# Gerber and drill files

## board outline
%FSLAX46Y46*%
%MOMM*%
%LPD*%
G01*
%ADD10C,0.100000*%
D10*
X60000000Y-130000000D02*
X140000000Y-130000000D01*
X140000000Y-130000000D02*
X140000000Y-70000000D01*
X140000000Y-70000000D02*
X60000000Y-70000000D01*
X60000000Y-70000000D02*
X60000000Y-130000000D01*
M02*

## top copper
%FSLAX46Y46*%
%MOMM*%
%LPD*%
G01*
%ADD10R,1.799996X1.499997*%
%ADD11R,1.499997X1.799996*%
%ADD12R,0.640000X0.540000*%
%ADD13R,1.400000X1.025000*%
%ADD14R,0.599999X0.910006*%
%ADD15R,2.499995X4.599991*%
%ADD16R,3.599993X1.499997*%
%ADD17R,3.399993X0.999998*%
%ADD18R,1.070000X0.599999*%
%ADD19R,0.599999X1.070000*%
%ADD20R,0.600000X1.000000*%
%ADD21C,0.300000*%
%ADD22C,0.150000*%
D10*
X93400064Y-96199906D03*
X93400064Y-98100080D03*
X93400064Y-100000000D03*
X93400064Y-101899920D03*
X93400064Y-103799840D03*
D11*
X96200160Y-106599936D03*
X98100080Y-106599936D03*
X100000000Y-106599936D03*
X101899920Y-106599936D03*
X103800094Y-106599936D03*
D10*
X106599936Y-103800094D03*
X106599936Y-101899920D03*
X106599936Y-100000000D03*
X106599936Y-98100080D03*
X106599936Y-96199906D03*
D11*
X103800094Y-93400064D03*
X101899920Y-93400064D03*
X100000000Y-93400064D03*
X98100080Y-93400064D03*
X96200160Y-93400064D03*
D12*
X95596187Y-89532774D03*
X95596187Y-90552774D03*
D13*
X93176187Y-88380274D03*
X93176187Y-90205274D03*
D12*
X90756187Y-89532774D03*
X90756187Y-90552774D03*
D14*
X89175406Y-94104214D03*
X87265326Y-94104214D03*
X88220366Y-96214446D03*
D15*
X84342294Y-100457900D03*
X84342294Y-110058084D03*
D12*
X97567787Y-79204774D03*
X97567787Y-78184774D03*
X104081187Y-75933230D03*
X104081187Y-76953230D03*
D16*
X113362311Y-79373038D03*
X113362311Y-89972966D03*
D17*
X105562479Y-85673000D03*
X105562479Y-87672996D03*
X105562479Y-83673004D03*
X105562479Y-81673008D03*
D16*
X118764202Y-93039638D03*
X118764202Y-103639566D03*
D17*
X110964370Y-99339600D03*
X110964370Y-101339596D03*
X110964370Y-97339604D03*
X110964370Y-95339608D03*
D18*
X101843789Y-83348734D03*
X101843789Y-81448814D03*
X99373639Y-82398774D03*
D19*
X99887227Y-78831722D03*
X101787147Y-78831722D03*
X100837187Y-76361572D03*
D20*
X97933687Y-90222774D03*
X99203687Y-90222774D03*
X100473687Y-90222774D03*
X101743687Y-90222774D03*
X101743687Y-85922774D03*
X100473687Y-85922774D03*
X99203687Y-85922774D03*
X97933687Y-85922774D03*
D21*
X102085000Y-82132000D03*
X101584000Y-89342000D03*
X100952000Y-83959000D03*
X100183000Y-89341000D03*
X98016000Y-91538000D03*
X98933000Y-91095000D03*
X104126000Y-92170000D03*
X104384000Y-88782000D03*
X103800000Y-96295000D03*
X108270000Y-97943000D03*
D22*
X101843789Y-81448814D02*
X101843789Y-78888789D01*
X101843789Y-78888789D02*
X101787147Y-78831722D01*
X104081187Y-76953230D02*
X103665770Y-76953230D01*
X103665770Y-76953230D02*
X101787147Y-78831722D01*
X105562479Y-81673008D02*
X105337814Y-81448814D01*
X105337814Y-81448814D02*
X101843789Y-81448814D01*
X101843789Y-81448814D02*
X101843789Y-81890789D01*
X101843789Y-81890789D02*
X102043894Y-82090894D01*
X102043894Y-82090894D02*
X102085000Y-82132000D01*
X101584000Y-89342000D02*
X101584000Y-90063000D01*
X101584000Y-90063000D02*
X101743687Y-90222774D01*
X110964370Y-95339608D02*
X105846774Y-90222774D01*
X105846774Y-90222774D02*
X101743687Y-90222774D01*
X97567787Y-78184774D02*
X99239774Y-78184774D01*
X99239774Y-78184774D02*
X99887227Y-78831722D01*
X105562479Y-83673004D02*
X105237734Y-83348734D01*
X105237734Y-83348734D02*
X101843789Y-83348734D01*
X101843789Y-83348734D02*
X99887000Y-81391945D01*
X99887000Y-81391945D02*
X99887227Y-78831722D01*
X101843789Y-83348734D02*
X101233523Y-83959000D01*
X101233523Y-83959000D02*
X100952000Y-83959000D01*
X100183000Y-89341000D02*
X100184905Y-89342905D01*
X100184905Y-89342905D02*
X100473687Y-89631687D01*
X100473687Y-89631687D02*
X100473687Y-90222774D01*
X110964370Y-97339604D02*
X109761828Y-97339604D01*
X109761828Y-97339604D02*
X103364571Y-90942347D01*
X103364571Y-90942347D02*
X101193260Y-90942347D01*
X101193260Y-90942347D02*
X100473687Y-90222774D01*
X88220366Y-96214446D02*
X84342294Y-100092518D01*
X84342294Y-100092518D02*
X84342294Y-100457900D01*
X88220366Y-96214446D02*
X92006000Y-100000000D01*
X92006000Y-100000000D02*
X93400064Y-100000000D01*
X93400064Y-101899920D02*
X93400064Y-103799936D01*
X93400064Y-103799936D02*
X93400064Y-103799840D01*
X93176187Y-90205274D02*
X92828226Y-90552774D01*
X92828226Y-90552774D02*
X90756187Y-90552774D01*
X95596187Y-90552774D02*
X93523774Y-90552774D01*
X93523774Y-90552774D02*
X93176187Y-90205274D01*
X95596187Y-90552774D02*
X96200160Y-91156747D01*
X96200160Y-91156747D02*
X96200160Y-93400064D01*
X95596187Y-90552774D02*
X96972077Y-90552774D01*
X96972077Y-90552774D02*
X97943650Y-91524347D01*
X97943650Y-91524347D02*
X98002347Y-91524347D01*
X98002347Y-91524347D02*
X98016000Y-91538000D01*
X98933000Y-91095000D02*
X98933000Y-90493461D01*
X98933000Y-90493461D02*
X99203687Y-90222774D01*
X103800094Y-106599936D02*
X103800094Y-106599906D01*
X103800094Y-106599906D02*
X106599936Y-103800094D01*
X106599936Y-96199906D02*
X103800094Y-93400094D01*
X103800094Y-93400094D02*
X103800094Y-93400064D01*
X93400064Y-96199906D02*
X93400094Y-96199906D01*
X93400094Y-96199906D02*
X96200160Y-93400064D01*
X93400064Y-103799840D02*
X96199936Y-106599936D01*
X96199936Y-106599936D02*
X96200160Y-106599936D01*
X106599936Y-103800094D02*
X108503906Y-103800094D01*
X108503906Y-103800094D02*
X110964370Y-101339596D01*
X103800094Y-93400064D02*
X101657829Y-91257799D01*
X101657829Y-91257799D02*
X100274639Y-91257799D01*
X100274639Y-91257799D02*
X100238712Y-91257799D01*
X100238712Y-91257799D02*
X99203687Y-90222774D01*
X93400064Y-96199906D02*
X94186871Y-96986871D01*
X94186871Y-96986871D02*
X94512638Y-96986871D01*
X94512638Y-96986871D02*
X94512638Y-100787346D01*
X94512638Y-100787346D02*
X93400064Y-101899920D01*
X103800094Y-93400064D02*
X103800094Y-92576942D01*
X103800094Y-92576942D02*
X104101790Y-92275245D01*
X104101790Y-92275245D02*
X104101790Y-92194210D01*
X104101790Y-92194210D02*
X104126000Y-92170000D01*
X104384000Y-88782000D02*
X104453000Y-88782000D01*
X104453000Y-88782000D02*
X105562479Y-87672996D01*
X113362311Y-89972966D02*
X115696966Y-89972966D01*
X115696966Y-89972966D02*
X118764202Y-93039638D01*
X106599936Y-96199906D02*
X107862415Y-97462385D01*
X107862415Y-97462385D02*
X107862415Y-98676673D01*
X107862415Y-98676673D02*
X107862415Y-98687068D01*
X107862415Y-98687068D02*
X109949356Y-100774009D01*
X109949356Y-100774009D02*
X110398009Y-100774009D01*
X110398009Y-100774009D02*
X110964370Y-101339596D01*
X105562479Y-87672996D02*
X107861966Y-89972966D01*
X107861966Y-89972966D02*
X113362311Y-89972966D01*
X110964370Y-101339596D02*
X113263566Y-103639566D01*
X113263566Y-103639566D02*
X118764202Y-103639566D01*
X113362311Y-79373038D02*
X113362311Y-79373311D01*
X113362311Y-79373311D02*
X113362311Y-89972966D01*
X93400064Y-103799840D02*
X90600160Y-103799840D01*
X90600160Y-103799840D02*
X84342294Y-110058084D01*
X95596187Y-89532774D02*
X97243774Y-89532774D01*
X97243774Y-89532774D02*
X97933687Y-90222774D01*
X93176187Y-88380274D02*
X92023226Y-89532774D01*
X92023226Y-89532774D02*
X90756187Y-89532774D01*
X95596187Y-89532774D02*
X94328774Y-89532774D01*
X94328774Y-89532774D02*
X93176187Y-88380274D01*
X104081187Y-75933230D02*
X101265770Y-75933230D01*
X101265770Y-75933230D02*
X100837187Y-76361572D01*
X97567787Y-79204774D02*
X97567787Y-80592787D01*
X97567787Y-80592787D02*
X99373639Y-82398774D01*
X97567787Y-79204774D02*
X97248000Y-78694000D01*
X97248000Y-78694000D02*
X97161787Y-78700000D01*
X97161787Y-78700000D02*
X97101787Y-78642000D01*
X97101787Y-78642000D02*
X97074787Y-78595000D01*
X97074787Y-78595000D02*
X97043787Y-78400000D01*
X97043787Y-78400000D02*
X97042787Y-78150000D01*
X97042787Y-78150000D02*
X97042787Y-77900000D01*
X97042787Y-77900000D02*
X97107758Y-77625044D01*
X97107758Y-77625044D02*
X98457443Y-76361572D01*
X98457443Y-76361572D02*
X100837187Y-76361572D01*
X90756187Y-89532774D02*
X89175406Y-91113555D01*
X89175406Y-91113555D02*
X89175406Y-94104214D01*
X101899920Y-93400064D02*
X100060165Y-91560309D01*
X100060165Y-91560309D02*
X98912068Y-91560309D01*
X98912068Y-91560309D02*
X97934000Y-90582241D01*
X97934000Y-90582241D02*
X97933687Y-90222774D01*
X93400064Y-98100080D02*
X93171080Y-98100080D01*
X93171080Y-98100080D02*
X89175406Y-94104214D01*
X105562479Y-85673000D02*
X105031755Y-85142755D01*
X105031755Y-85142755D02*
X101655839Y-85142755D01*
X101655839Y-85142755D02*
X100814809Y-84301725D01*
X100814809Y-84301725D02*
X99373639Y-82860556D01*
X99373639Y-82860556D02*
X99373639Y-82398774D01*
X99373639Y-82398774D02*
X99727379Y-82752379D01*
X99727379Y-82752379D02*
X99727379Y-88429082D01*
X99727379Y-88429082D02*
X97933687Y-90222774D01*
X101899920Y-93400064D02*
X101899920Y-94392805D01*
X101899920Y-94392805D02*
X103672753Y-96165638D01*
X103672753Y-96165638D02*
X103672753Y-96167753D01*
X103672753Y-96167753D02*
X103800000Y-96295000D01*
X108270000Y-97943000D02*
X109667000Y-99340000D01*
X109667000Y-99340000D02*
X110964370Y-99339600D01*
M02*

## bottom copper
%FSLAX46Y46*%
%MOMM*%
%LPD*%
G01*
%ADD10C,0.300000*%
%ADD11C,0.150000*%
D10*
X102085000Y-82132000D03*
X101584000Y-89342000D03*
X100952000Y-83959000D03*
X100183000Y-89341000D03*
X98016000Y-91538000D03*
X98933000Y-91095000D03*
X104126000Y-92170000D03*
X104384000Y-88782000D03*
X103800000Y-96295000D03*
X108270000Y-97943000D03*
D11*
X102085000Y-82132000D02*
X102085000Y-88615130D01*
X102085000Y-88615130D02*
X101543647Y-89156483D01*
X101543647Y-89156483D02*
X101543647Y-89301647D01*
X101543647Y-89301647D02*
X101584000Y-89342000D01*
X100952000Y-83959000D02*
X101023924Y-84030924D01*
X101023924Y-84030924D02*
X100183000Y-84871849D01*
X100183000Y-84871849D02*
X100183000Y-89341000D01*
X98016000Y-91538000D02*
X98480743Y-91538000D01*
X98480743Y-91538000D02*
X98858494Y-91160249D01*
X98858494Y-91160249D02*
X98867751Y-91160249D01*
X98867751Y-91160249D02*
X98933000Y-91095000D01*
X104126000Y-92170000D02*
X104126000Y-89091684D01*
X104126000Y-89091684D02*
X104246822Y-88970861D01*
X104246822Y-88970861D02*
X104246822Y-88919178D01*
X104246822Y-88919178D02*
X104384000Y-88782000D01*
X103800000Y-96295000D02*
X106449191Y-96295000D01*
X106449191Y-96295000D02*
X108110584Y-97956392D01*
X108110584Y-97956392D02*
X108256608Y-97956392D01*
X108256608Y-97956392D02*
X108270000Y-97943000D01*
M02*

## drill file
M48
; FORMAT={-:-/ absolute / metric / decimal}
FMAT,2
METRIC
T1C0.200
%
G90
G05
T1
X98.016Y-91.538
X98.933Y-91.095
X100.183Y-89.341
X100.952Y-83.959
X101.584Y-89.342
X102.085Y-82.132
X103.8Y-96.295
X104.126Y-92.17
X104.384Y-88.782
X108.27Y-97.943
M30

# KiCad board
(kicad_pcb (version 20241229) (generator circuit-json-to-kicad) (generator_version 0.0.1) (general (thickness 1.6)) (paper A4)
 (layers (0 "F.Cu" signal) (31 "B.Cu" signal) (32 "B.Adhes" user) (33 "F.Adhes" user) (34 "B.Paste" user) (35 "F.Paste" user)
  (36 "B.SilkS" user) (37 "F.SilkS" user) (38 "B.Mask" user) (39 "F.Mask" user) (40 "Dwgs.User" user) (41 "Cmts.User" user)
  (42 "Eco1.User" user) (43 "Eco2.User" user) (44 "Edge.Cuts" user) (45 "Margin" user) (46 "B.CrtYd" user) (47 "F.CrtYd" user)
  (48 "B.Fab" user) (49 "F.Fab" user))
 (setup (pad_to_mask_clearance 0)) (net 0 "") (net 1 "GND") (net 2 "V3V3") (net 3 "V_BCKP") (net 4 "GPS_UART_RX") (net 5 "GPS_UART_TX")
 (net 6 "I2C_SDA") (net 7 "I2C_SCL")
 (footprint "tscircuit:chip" (layer F.Cu) (at 100 100 0)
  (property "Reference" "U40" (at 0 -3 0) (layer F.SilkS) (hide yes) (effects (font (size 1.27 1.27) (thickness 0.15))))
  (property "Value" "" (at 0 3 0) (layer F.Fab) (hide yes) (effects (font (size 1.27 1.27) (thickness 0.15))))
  (pad "1" smd rect (at -6.5999360000001275 -3.8000939999998877 0) (size 1.7999964 1.499997) (layers F.Cu F.Paste F.Mask) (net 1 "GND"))
  (pad "2" smd rect (at -6.5999360000001275 -1.899919999999895 0) (size 1.7999964 1.499997) (layers F.Cu F.Paste F.Mask) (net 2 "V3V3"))
  (pad "3" smd rect (at -6.5999360000001275 5.684341886080802e-14 0) (size 1.7999964 1.499997) (layers F.Cu F.Paste F.Mask) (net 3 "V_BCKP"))
  (pad "4" smd rect (at -6.5999360000001275 1.8999200000000087 0) (size 1.7999964 1.499997) (layers F.Cu F.Paste F.Mask) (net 1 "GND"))
  (pad "5" smd rect (at -6.5999360000001275 3.7998400000000743 0) (size 1.7999964 1.499997) (layers F.Cu F.Paste F.Mask) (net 1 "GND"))
  (pad "6" smd rect (at -3.7998399999999606 6.599936000000014 0) (size 1.499997 1.7999964) (layers F.Cu F.Paste F.Mask) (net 1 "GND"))
  (pad "7" smd rect (at -1.899919999999895 6.599936000000014 0) (size 1.499997 1.7999964) (layers F.Cu F.Paste F.Mask))
  (pad "8" smd rect (at -5.684341886080802e-14 6.599936000000014 0) (size 1.499997 1.7999964) (layers F.Cu F.Paste F.Mask))
  (pad "9" smd rect (at 1.899919999999895 6.599936000000014 0) (size 1.499997 1.7999964) (layers F.Cu F.Paste F.Mask))
  (pad "10" smd rect (at 3.8000940000000014 6.599936000000014 0) (size 1.499997 1.7999964) (layers F.Cu F.Paste F.Mask) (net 1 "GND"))
  (pad "11" smd rect (at 6.5999360000001275 3.800094000000115 0) (size 1.7999964 1.499997) (layers F.Cu F.Paste F.Mask) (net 1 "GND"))
  (pad "12" smd rect (at 6.5999360000001275 1.8999200000000087 0) (size 1.7999964 1.499997) (layers F.Cu F.Paste F.Mask))
  (pad "13" smd rect (at 6.5999360000001275 5.684341886080802e-14 0) (size 1.7999964 1.499997) (layers F.Cu F.Paste F.Mask)
   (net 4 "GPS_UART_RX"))
  (pad "14" smd rect (at 6.5999360000001275 -1.899919999999895 0) (size 1.7999964 1.499997) (layers F.Cu F.Paste F.Mask)
   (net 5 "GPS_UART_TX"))
  (pad "15" smd rect (at 6.5999360000001275 -3.8000939999998877 0) (size 1.7999964 1.499997) (layers F.Cu F.Paste F.Mask) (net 1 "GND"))
  (pad "16" smd rect (at 3.8000940000000014 -6.599936000000014 0) (size 1.499997 1.7999964) (layers F.Cu F.Paste F.Mask) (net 1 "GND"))
  (pad "17" smd rect (at 1.899919999999895 -6.599936000000014 0) (size 1.499997 1.7999964) (layers F.Cu F.Paste F.Mask) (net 2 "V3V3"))
  (pad "18" smd rect (at -5.684341886080802e-14 -6.599936000000014 0) (size 1.499997 1.7999964) (layers F.Cu F.Paste F.Mask))
  (pad "19" smd rect (at -1.899919999999895 -6.599936000000014 0) (size 1.499997 1.7999964) (layers F.Cu F.Paste F.Mask))
  (pad "20" smd rect (at -3.7998399999999606 -6.599936000000014 0) (size 1.499997 1.7999964) (layers F.Cu F.Paste F.Mask) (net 1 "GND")))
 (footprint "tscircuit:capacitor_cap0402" (layer F.Cu) (at 95.59618690909089 90.04277400000001 -90.00000000000001)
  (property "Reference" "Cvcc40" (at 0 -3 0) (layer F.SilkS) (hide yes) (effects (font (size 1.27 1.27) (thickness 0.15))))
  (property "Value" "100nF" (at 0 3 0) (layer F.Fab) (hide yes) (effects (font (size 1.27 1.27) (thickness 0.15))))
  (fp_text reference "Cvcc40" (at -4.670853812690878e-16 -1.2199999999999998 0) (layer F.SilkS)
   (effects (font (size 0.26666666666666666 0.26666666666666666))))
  (pad "1" smd rect (at -0.5099999999999998 8.881784197001252e-16 0) (size 0.64 0.54) (layers F.Cu F.Paste F.Mask) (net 2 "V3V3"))
  (pad "2" smd rect (at 0.5099999999999998 0 0) (size 0.64 0.54) (layers F.Cu F.Paste F.Mask) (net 1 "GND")))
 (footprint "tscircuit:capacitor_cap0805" (layer F.Cu) (at 93.17618690909089 89.29277400000001 -90.00000000000001)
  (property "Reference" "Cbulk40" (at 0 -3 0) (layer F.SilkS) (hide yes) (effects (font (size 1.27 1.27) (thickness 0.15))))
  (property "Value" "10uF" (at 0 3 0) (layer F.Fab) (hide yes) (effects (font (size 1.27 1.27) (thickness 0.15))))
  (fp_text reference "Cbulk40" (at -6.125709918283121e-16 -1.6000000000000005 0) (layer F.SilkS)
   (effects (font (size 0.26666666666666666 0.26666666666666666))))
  (pad "1" smd rect (at -0.9124999999999996 0 0) (size 1.4 1.025) (layers F.Cu F.Paste F.Mask) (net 2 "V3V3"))
  (pad "2" smd rect (at 0.9124999999999996 -8.881784197001252e-16 0) (size 1.4 1.025) (layers F.Cu F.Paste F.Mask) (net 1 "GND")))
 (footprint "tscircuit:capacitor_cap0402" (layer F.Cu) (at 90.75618690909089 90.04277400000001 -90.00000000000001)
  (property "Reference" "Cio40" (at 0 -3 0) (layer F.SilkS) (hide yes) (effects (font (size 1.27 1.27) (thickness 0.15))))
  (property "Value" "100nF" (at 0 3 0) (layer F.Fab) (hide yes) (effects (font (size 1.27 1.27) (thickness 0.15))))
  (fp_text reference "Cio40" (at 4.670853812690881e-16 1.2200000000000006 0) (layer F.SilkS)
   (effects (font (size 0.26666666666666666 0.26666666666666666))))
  (pad "1" smd rect (at -0.5099999999999998 0 0) (size 0.64 0.54) (layers F.Cu F.Paste F.Mask) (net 2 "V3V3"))
  (pad "2" smd rect (at 0.5099999999999998 0 0) (size 0.64 0.54) (layers F.Cu F.Paste F.Mask) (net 1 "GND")))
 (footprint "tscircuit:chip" (layer F.Cu) (at 88.22036600000001 95.15933033333334 90)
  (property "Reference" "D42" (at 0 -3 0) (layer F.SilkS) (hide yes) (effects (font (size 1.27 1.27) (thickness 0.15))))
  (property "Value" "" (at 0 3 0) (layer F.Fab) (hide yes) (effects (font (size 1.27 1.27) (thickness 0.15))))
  (pad "1" smd rect (at 1.0551160000000053 0.9550400000000039 0) (size 0.5999987999999999 0.9100057999999999) (layers F.Cu F.Paste F.Mask)
   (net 2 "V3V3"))
  (pad "2" smd rect (at 1.0551160000000053 -0.9550400000000039 0) (size 0.5999987999999999 0.9100057999999999) (layers F.Cu F.Paste F.Mask))
  (pad "3" smd rect (at -1.0551160000000053 7.105427357601002e-15 0) (size 0.5999987999999999 0.9100057999999999)
   (layers F.Cu F.Paste F.Mask) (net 3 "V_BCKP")))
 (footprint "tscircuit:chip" (layer F.Cu) (at 84.34229399999987 105.25799233333349 -90.00000000000001)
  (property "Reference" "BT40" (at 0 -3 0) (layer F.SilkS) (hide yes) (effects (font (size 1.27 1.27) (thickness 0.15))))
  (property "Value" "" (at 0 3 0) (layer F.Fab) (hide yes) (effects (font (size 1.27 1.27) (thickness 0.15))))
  (pad "1" smd rect (at -4.80009200000012 1.7763568394002505e-15 0) (size 2.4999949999999997 4.5999908) (layers F.Cu F.Paste F.Mask)
   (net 3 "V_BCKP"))
  (pad "2" smd rect (at 4.800092000000118 -1.7763568394002505e-15 0) (size 2.4999949999999997 4.5999908) (layers F.Cu F.Paste F.Mask)
   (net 1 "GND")))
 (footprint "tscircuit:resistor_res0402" (layer F.Cu) (at 97.5677869090909 78.69477400000001 90)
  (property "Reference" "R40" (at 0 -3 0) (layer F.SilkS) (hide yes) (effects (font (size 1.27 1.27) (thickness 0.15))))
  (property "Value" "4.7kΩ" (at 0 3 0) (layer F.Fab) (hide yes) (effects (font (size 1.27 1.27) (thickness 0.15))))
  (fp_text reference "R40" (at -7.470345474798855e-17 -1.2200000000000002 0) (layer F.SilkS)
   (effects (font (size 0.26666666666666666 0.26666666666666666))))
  (pad "1" smd rect (at -0.5100000000000016 0 0) (size 0.64 0.54) (layers F.Cu F.Paste F.Mask) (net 2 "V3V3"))
  (pad "2" smd rect (at 0.5100000000000016 0 0) (size 0.64 0.54) (layers F.Cu F.Paste F.Mask) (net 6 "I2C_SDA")))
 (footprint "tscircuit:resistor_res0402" (layer F.Cu) (at 104.08118690909089 76.44322999999997 -90.00000000000001)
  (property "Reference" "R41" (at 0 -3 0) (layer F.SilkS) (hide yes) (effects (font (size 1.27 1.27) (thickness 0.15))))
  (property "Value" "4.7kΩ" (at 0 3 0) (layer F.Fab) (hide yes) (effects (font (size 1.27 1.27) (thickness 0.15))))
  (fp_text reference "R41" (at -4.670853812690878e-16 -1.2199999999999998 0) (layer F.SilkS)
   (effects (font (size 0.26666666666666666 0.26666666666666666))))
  (pad "1" smd rect (at -0.5100000000000016 0 0) (size 0.64 0.54) (layers F.Cu F.Paste F.Mask) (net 2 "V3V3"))
  (pad "2" smd rect (at 0.5100000000000016 0 0) (size 0.64 0.54) (layers F.Cu F.Paste F.Mask) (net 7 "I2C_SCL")))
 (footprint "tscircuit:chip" (layer F.Cu) (at 109.51239480909098 84.673002 90)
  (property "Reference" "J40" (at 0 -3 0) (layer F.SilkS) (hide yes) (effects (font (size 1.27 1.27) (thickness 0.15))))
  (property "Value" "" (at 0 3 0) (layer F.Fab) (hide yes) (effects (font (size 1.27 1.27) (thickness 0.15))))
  (pad "5" smd rect (at 5.299963999999989 3.8499161000000193 0) (size 3.5999928 1.499997) (layers F.Cu F.Paste F.Mask) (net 1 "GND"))
  (pad "6" smd rect (at -5.299963999999989 3.849916100000021 0) (size 3.5999928 1.499997) (layers F.Cu F.Paste F.Mask) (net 1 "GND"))
  (pad "2" smd rect (at -0.9999979999999482 -3.9499159000000175 0) (size 3.3999932 0.9999979999999999) (layers F.Cu F.Paste F.Mask)
   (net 2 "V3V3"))
  (pad "1" smd rect (at -2.999994000000072 -3.9499159000000175 0) (size 3.3999932 0.9999979999999999) (layers F.Cu F.Paste F.Mask)
   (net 1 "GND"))
  (pad "3" smd rect (at 0.9999979999999482 -3.9499159000000175 0) (size 3.3999932 0.9999979999999999) (layers F.Cu F.Paste F.Mask)
   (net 6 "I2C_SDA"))
  (pad "4" smd rect (at 2.9999939999999583 -3.9499159000000175 0) (size 3.3999932 0.9999979999999999) (layers F.Cu F.Paste F.Mask)
   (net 7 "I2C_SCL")))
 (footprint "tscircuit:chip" (layer F.Cu) (at 114.9142860999999 98.33960200000001 90)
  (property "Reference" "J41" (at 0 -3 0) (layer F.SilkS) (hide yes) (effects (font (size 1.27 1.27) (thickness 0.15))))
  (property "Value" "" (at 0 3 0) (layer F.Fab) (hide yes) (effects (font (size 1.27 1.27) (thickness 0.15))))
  (pad "5" smd rect (at 5.299963999999989 3.8499161000000193 0) (size 3.5999928 1.499997) (layers F.Cu F.Paste F.Mask) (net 1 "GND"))
  (pad "6" smd rect (at -5.299963999999989 3.8499161000000193 0) (size 3.5999928 1.499997) (layers F.Cu F.Paste F.Mask) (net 1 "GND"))
  (pad "2" smd rect (at -0.9999979999999482 -3.9499159000000184 0) (size 3.3999932 0.9999979999999999) (layers F.Cu F.Paste F.Mask)
   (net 2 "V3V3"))
  (pad "1" smd rect (at -2.999994000000072 -3.9499159000000184 0) (size 3.3999932 0.9999979999999999) (layers F.Cu F.Paste F.Mask)
   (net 1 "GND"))
  (pad "3" smd rect (at 0.9999979999999482 -3.9499159000000184 0) (size 3.3999932 0.9999979999999999) (layers F.Cu F.Paste F.Mask)
   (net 6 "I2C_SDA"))
  (pad "4" smd rect (at 2.9999939999999583 -3.9499159000000184 0) (size 3.3999932 0.9999979999999999) (layers F.Cu F.Paste F.Mask)
   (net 7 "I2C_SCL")))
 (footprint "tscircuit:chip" (layer F.Cu) (at 100.60871390909071 82.39877400000002 0)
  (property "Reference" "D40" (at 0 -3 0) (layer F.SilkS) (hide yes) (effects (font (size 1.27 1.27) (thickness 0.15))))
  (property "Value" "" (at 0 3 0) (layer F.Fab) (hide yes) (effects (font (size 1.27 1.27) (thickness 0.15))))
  (pad "1" smd rect (at 1.2350749999999948 0.9499599999999191 0) (size 1.0700004 0.5999987999999999) (layers F.Cu F.Paste F.Mask)
   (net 6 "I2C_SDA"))
  (pad "2" smd rect (at 1.2350749999999948 -0.9499599999999191 0) (size 1.0700004 0.5999987999999999) (layers F.Cu F.Paste F.Mask)
   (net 7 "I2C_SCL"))
  (pad "3" smd rect (at -1.2350749999999948 0 0) (size 1.0700004 0.5999987999999999) (layers F.Cu F.Paste F.Mask) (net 2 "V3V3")))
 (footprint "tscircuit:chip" (layer F.Cu) (at 100.83718690909089 77.59664700000003 -90.00000000000001)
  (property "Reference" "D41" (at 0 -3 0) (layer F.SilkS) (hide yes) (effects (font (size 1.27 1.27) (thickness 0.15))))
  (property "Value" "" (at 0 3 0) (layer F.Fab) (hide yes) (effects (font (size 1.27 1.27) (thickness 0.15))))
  (pad "1" smd rect (at 1.2350749999999948 0.9499599999999189 0) (size 0.5999987999999999 1.0700004) (layers F.Cu F.Paste F.Mask)
   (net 6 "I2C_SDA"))
  (pad "2" smd rect (at 1.2350749999999948 -0.9499599999999194 0) (size 0.5999987999999999 1.0700004) (layers F.Cu F.Paste F.Mask)
   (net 7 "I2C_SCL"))
  (pad "3" smd rect (at -1.2350749999999948 3.3306690738754696e-16 0) (size 0.5999987999999999 1.0700004) (layers F.Cu F.Paste F.Mask)
   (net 2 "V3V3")))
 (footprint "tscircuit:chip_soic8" (layer F.Cu) (at 99.83868690909088 88.07277400000001 90)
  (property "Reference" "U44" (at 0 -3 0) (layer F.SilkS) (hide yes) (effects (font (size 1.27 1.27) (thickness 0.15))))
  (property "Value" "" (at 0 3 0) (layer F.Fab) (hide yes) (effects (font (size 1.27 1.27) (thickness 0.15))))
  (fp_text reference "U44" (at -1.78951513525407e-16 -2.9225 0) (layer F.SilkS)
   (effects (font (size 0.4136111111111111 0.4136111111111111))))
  (pad "1" smd rect (at -2.1500000000000004 -1.905 0) (size 0.6 1) (layers F.Cu F.Paste F.Mask) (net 2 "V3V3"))
  (pad "2" smd rect (at -2.1500000000000004 -0.635 0) (size 0.6 1) (layers F.Cu F.Paste F.Mask) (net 1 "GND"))
  (pad "3" smd rect (at -2.1500000000000004 0.635 0) (size 0.6 1) (layers F.Cu F.Paste F.Mask) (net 6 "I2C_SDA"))
  (pad "4" smd rect (at -2.1500000000000004 1.9049999999999998 0) (size 0.6 1) (layers F.Cu F.Paste F.Mask) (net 7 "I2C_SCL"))
  (pad "5" smd rect (at 2.1500000000000004 1.905 0) (size 0.6 1) (layers F.Cu F.Paste F.Mask))
  (pad "6" smd rect (at 2.1500000000000004 0.635 0) (size 0.6 1) (layers F.Cu F.Paste F.Mask))
  (pad "7" smd rect (at 2.1500000000000004 -0.635 0) (size 0.6 1) (layers F.Cu F.Paste F.Mask))
  (pad "8" smd rect (at 2.1500000000000004 -1.905 0) (size 0.6 1) (layers F.Cu F.Paste F.Mask)))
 (segment (start 101.8437889090907 81.4488140000001) (end 101.8437889090907 78.8887889090907) (width 0.15) (layer F.Cu) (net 7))
 (segment (start 101.8437889090907 78.8887889090907) (end 101.78714690909081 78.83172200000003) (width 0.15) (layer F.Cu) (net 7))
 (segment (start 104.08118690909089 76.95322999999998) (end 103.66577000000002 76.95322999999998) (width 0.15) (layer F.Cu) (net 7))
 (segment (start 103.66577000000002 76.95322999999998) (end 101.78714690909081 78.83172200000003) (width 0.15) (layer F.Cu) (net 7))
 (segment (start 105.56247890909097 81.67300800000004) (end 105.3378140000001 81.4488140000001) (width 0.15) (layer F.Cu) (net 7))
 (segment (start 105.3378140000001 81.4488140000001) (end 101.8437889090907 81.4488140000001) (width 0.15) (layer F.Cu) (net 7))
 (segment (start 101.8437889090907 81.4488140000001) (end 101.8437889090907 81.8907889090907) (width 0.15) (layer F.Cu) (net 7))
 (segment (start 101.8437889090907 81.8907889090907) (end 102.04389361014476 82.09089361014476) (width 0.15) (layer F.Cu) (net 7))
 (segment (start 102.04389361014476 82.09089361014476) (end 102.085 82.132) (width 0.15) (layer F.Cu) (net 7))
 (segment (start 102.085 82.132) (end 102.085 88.61512961316996) (width 0.15) (layer B.Cu) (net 7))
 (segment (start 102.085 88.61512961316996) (end 101.54364677566849 89.15648283750146) (width 0.15) (layer B.Cu) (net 7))
 (segment (start 101.54364677566849 89.15648283750146) (end 101.54364677566849 89.30164677566849) (width 0.15) (layer B.Cu) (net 7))
 (segment (start 101.54364677566849 89.30164677566849) (end 101.584 89.342) (width 0.15) (layer B.Cu) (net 7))
 (segment (start 101.584 89.342) (end 101.584 90.063) (width 0.15) (layer F.Cu) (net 7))
 (segment (start 101.584 90.063) (end 101.74368690909088 90.22277400000002) (width 0.15) (layer F.Cu) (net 7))
 (segment (start 110.96437019999988 95.33960800000006) (end 105.84677400000001 90.22277400000002) (width 0.15) (layer F.Cu) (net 7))
 (segment (start 105.84677400000001 90.22277400000002) (end 101.74368690909088 90.22277400000002) (width 0.15) (layer F.Cu) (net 7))
 (segment (start 97.5677869090909 78.184774) (end 99.23977400000001 78.184774) (width 0.15) (layer F.Cu) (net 6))
 (segment (start 99.23977400000001 78.184774) (end 99.88722690909097 78.83172200000003) (width 0.15) (layer F.Cu) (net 6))
 (segment (start 105.56247890909097 83.67300400000005) (end 105.23773399999993 83.34873399999994) (width 0.15) (layer F.Cu) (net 6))
 (segment (start 105.23773399999993 83.34873399999994) (end 101.8437889090907 83.34873399999994) (width 0.15) (layer F.Cu) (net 6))
 (segment (start 101.8437889090907 83.34873399999994) (end 99.887 81.39194509090923) (width 0.15) (layer F.Cu) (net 6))
 (segment (start 99.887 81.39194509090923) (end 99.88722690909097 78.83172200000003) (width 0.15) (layer F.Cu) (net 6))
 (segment (start 101.8437889090907 83.34873399999994) (end 101.23352290909064 83.959) (width 0.15) (layer F.Cu) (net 6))
 (segment (start 101.23352290909064 83.959) (end 100.952 83.959) (width 0.15) (layer F.Cu) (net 6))
 (segment (start 100.952 83.959) (end 101.02392440211129 84.0309244021113) (width 0.15) (layer B.Cu) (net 6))
 (segment (start 101.02392440211129 84.0309244021113) (end 100.183 84.87184880422258) (width 0.15) (layer B.Cu) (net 6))
 (segment (start 100.183 84.87184880422258) (end 100.183 89.341) (width 0.15) (layer B.Cu) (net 6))
 (segment (start 100.183 89.341) (end 100.18490502715771 89.34290502715771) (width 0.15) (layer F.Cu) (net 6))
 (segment (start 100.18490502715771 89.34290502715771) (end 100.47368690909089 89.63168690909089) (width 0.15) (layer F.Cu) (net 6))
 (segment (start 100.47368690909089 89.63168690909089) (end 100.47368690909089 90.22277400000002) (width 0.15) (layer F.Cu) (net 6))
 (segment (start 110.96437019999988 97.33960400000007) (end 109.76182780906325 97.33960400000007) (width 0.15) (layer F.Cu) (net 6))
 (segment (start 109.76182780906325 97.33960400000007) (end 103.36457059215748 90.9423467830943) (width 0.15) (layer F.Cu) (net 6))
 (segment (start 103.36457059215748 90.9423467830943) (end 101.19325969218517 90.9423467830943) (width 0.15) (layer F.Cu) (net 6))
 (segment (start 101.19325969218517 90.9423467830943) (end 100.47368690909089 90.22277400000002) (width 0.15) (layer F.Cu) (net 6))
 (segment (start 88.22036600000003 96.21444633333336) (end 84.34229399999987 100.09251833333352) (width 0.15) (layer F.Cu) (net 3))
 (segment (start 84.34229399999987 100.09251833333352) (end 84.34229399999987 100.45790033333337) (width 0.15) (layer F.Cu) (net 3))
 (segment (start 88.22036600000003 96.21444633333336) (end 92.00600000000006 100.00000000000006) (width 0.15) (layer F.Cu) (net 3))
 (segment (start 92.00600000000006 100.00000000000006) (end 93.40006399999987 100.00000000000006) (width 0.15) (layer F.Cu) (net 3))
 (segment (start 93.40006399999987 101.89992000000001) (end 93.40006399999987 103.79993600000013) (width 0.15) (layer F.Cu) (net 1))
 (segment (start 93.40006399999987 103.79993600000013) (end 93.40006399999987 103.79984000000007) (width 0.15) (layer F.Cu) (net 1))
 (segment (start 93.17618690909089 90.20527400000002) (end 92.82822599999999 90.55277400000001) (width 0.15) (layer F.Cu) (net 1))
 (segment (start 92.82822599999999 90.55277400000001) (end 90.75618690909089 90.55277400000001) (width 0.15) (layer F.Cu) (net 1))
 (segment (start 95.59618690909089 90.55277400000001) (end 93.52377400000002 90.55277400000001) (width 0.15) (layer F.Cu) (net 1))
 (segment (start 93.52377400000002 90.55277400000001) (end 93.17618690909089 90.20527400000002) (width 0.15) (layer F.Cu) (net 1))
 (segment (start 95.59618690909089 90.55277400000001) (end 96.20016000000004 91.15674709090916) (width 0.15) (layer F.Cu) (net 1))
 (segment (start 96.20016000000004 91.15674709090916) (end 96.20016000000004 93.40006399999999) (width 0.15) (layer F.Cu) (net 1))
 (segment (start 95.59618690909089 90.55277400000001) (end 96.9720768660011 90.55277400000001) (width 0.15) (layer F.Cu) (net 1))
 (segment (start 96.9720768660011 90.55277400000001) (end 97.9436502400804 91.52434737407931) (width 0.15) (layer F.Cu) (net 1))
 (segment (start 97.9436502400804 91.52434737407931) (end 98.00234737407932 91.52434737407931) (width 0.15) (layer F.Cu) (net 1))
 (segment (start 98.00234737407932 91.52434737407931) (end 98.016 91.538) (width 0.15) (layer F.Cu) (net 1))
 (segment (start 98.016 91.538) (end 98.48074301078097 91.538) (width 0.15) (layer B.Cu) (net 1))
 (segment (start 98.48074301078097 91.538) (end 98.85849426996063 91.16024874082035) (width 0.15) (layer B.Cu) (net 1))
 (segment (start 98.85849426996063 91.16024874082035) (end 98.86775125917966 91.16024874082035) (width 0.15) (layer B.Cu) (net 1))
 (segment (start 98.86775125917966 91.16024874082035) (end 98.933 91.095) (width 0.15) (layer B.Cu) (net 1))
 (segment (start 98.933 91.095) (end 98.933 90.4934609090909) (width 0.15) (layer F.Cu) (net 1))
 (segment (start 98.933 90.4934609090909) (end 99.20368690909089 90.22277400000002) (width 0.15) (layer F.Cu) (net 1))
 (segment (start 103.800094 106.59993600000001) (end 103.800094 106.599906) (width 0.15) (layer F.Cu) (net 1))
 (segment (start 103.800094 106.599906) (end 106.59993600000013 103.80009400000012) (width 0.15) (layer F.Cu) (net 1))
 (segment (start 106.59993600000013 96.19990600000011) (end 103.800094 93.400094) (width 0.15) (layer F.Cu) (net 1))
 (segment (start 103.800094 93.400094) (end 103.800094 93.40006399999999) (width 0.15) (layer F.Cu) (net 1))
 (segment (start 93.40006399999987 96.19990600000011) (end 93.40009399999988 96.19990600000011) (width 0.15) (layer F.Cu) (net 1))
 (segment (start 93.40009399999988 96.19990600000011) (end 96.20016000000004 93.40006399999999) (width 0.15) (layer F.Cu) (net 1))
 (segment (start 93.40006399999987 103.79984000000007) (end 96.19993600000001 106.59993600000001) (width 0.15) (layer F.Cu) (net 1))
 (segment (start 96.19993600000001 106.59993600000001) (end 96.20016000000004 106.59993600000001) (width 0.15) (layer F.Cu) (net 1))
 (segment (start 106.59993600000013 103.80009400000012) (end 108.50390599999989 103.80009400000012) (width 0.15) (layer F.Cu) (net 1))
 (segment (start 108.50390599999989 103.80009400000012) (end 110.96437019999988 101.33959600000009) (width 0.15) (layer F.Cu) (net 1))
 (segment (start 103.800094 93.40006399999999) (end 101.65782904262174 91.25779904262173) (width 0.15) (layer F.Cu) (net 1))
 (segment (start 101.65782904262174 91.25779904262173) (end 100.27463858545984 91.25779904262173) (width 0.15) (layer F.Cu) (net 1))
 (segment (start 100.27463858545984 91.25779904262173) (end 100.2387119517126 91.25779904262173) (width 0.15) (layer F.Cu) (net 1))
 (segment (start 100.2387119517126 91.25779904262173) (end 99.20368690909089 90.22277400000002) (width 0.15) (layer F.Cu) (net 1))
 (segment (start 93.40006399999987 96.19990600000011) (end 94.18687091737846 96.98687091737845) (width 0.15) (layer F.Cu) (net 1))
 (segment (start 94.18687091737846 96.98687091737845) (end 94.51263838721975 96.98687091737845) (width 0.15) (layer F.Cu) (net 1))
 (segment (start 94.51263838721975 96.98687091737845) (end 94.51263838721975 100.78734561278013) (width 0.15) (layer F.Cu) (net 1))
 (segment (start 94.51263838721975 100.78734561278013) (end 93.40006399999987 101.89992000000001) (width 0.15) (layer F.Cu) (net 1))
 (segment (start 103.800094 93.40006399999999) (end 103.800094 92.57694157541104) (width 0.15) (layer F.Cu) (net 1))
 (segment (start 103.800094 92.57694157541104) (end 104.10179022764605 92.27524534776501) (width 0.15) (layer F.Cu) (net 1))
 (segment (start 104.10179022764605 92.27524534776501) (end 104.10179022764605 92.19420977235396) (width 0.15) (layer F.Cu) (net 1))
 (segment (start 104.10179022764605 92.19420977235396) (end 104.126 92.17) (width 0.15) (layer F.Cu) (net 1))
 (segment (start 104.126 92.17) (end 104.126 89.09168353513688) (width 0.15) (layer B.Cu) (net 1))
 (segment (start 104.126 89.09168353513688) (end 104.24682231012956 88.97086122500733) (width 0.15) (layer B.Cu) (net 1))
 (segment (start 104.24682231012956 88.97086122500733) (end 104.24682231012956 88.91917768987045) (width 0.15) (layer B.Cu) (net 1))
 (segment (start 104.24682231012956 88.91917768987045) (end 104.384 88.782) (width 0.15) (layer B.Cu) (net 1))
 (segment (start 104.384 88.782) (end 104.453 88.782) (width 0.15) (layer F.Cu) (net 1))
 (segment (start 104.453 88.782) (end 105.56247890909097 87.67299600000007) (width 0.15) (layer F.Cu) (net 1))
 (segment (start 113.36231090909101 89.97296599999999) (end 115.69696599999999 89.97296599999999) (width 0.15) (layer F.Cu) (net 1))
 (segment (start 115.69696599999999 89.97296599999999) (end 118.76420219999991 93.03963800000002) (width 0.15) (layer F.Cu) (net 1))
 (segment (start 106.59993600000013 96.19990600000011) (end 107.86241542483387 97.46238542483385) (width 0.15) (layer F.Cu) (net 1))
 (segment (start 107.86241542483387 97.46238542483385) (end 107.86241542483387 98.67667293813103) (width 0.15) (layer F.Cu) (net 1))
 (segment (start 107.86241542483387 98.67667293813103) (end 107.86241542483387 98.68706794518017) (width 0.15) (layer F.Cu) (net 1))
 (segment (start 107.86241542483387 98.68706794518017) (end 109.9493563308026 100.77400885114889) (width 0.15) (layer F.Cu) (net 1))
 (segment (start 109.9493563308026 100.77400885114889) (end 110.39800885114889 100.77400885114889) (width 0.15) (layer F.Cu) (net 1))
 (segment (start 110.39800885114889 100.77400885114889) (end 110.96437019999988 101.33959600000009) (width 0.15) (layer F.Cu) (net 1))
 (segment (start 105.56247890909097 87.67299600000007) (end 107.86196599999998 89.97296599999999) (width 0.15) (layer F.Cu) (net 1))
 (segment (start 107.86196599999998 89.97296599999999) (end 113.36231090909101 89.97296599999999) (width 0.15) (layer F.Cu) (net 1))
 (segment (start 110.96437019999988 101.33959600000009) (end 113.263566 103.639566) (width 0.15) (layer F.Cu) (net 1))
 (segment (start 113.263566 103.639566) (end 118.76420219999991 103.639566) (width 0.15) (layer F.Cu) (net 1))
 (segment (start 113.36231090909101 79.37303800000001) (end 113.36231090909101 79.373310909091) (width 0.15) (layer F.Cu) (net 1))
 (segment (start 113.36231090909101 79.373310909091) (end 113.36231090909101 89.97296599999999) (width 0.15) (layer F.Cu) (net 1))
 (segment (start 93.40006399999987 103.79984000000007) (end 90.60015999999993 103.79984000000007) (width 0.15) (layer F.Cu) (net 1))
 (segment (start 90.60015999999993 103.79984000000007) (end 84.34229399999987 110.05808433333361) (width 0.15) (layer F.Cu) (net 1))
 (segment (start 95.59618690909089 89.53277400000002) (end 97.24377400000002 89.53277400000002) (width 0.15) (layer F.Cu) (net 2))
 (segment (start 97.24377400000002 89.53277400000002) (end 97.93368690909088 90.22277400000002) (width 0.15) (layer F.Cu) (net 2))
 (segment (start 93.17618690909089 88.38027400000001) (end 92.02322599999998 89.53277400000002) (width 0.15) (layer F.Cu) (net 2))
 (segment (start 92.02322599999998 89.53277400000002) (end 90.75618690909089 89.53277400000002) (width 0.15) (layer F.Cu) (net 2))
 (segment (start 95.59618690909089 89.53277400000002) (end 94.32877400000001 89.53277400000002) (width 0.15) (layer F.Cu) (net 2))
 (segment (start 94.32877400000001 89.53277400000002) (end 93.17618690909089 88.38027400000001) (width 0.15) (layer F.Cu) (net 2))
 (segment (start 104.08118690909089 75.93322999999998) (end 101.26577000000002 75.93322999999998) (width 0.15) (layer F.Cu) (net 2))
 (segment (start 101.26577000000002 75.93322999999998) (end 100.83718690909089 76.36157200000004) (width 0.15) (layer F.Cu) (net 2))
 (segment (start 97.5677869090909 79.20477400000001) (end 97.5677869090909 80.59278690909089) (width 0.15) (layer F.Cu) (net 2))
 (segment (start 97.5677869090909 80.59278690909089) (end 99.37363890909072 82.39877400000002) (width 0.15) (layer F.Cu) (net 2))
 (segment (start 97.5677869090909 79.20477400000001) (end 97.248 78.694) (width 0.15) (layer F.Cu) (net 2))
 (segment (start 97.248 78.694) (end 97.16178690909089 78.7) (width 0.15) (layer F.Cu) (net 2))
 (segment (start 97.16178690909089 78.7) (end 97.10178690909089 78.642) (width 0.15) (layer F.Cu) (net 2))
 (segment (start 97.10178690909089 78.642) (end 97.07478690909089 78.595) (width 0.15) (layer F.Cu) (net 2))
 (segment (start 97.07478690909089 78.595) (end 97.0437869090909 78.4) (width 0.15) (layer F.Cu) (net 2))
 (segment (start 97.0437869090909 78.4) (end 97.04278690909089 78.15) (width 0.15) (layer F.Cu) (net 2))
 (segment (start 97.04278690909089 78.15) (end 97.04278690909089 77.9) (width 0.15) (layer F.Cu) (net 2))
 (segment (start 97.04278690909089 77.9) (end 97.10775795964962 77.62504380483477) (width 0.15) (layer F.Cu) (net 2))
 (segment (start 97.10775795964962 77.62504380483477) (end 98.45744285539348 76.36157200000004) (width 0.15) (layer F.Cu) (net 2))
 (segment (start 98.45744285539348 76.36157200000004) (end 100.83718690909089 76.36157200000004) (width 0.15) (layer F.Cu) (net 2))
 (segment (start 90.75618690909089 89.53277400000002) (end 89.17540600000002 91.11355490909088) (width 0.15) (layer F.Cu) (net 2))
 (segment (start 89.17540600000002 91.11355490909088) (end 89.17540600000002 94.10421433333335) (width 0.15) (layer F.Cu) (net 2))
 (segment (start 101.8999199999999 93.40006399999999) (end 100.06016537717214 91.56030937717223) (width 0.15) (layer F.Cu) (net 2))
 (segment (start 100.06016537717214 91.56030937717223) (end 98.91206788137922 91.56030937717223) (width 0.15) (layer F.Cu) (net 2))
 (segment (start 98.91206788137922 91.56030937717223) (end 97.934 90.58224149579303) (width 0.15) (layer F.Cu) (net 2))
 (segment (start 97.934 90.58224149579303) (end 97.93368690909088 90.22277400000002) (width 0.15) (layer F.Cu) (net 2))
 (segment (start 93.40006399999987 98.1000800000001) (end 93.1710800000001 98.1000800000001) (width 0.15) (layer F.Cu) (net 2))
 (segment (start 93.1710800000001 98.1000800000001) (end 89.17540600000002 94.10421433333335) (width 0.15) (layer F.Cu) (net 2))
 (segment (start 105.56247890909097 85.67299999999994) (end 105.03175519427019 85.1427551942702) (width 0.15) (layer F.Cu) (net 2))
 (segment (start 105.03175519427019 85.1427551942702) (end 101.65583853323 85.1427551942702) (width 0.15) (layer F.Cu) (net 2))
 (segment (start 101.65583853323 85.1427551942702) (end 100.8148087481819 84.3017254092221) (width 0.15) (layer F.Cu) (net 2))
 (segment (start 100.8148087481819 84.3017254092221) (end 99.37363890909072 82.8605555701309) (width 0.15) (layer F.Cu) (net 2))
 (segment (start 99.37363890909072 82.8605555701309) (end 99.37363890909072 82.39877400000002) (width 0.15) (layer F.Cu) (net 2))
 (segment (start 99.37363890909072 82.39877400000002) (end 99.72737938894376 82.75237938894375) (width 0.15) (layer F.Cu) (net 2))
 (segment (start 99.72737938894376 82.75237938894375) (end 99.72737938894376 88.42908152014714) (width 0.15) (layer F.Cu) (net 2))
 (segment (start 99.72737938894376 88.42908152014714) (end 97.93368690909088 90.22277400000002) (width 0.15) (layer F.Cu) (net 2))
 (segment (start 101.8999199999999 93.40006399999999) (end 101.8999199999999 94.39280520285473) (width 0.15) (layer F.Cu) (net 2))
 (segment (start 101.8999199999999 94.39280520285473) (end 103.67275319370076 96.16563839655561) (width 0.15) (layer F.Cu) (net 2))
 (segment (start 103.67275319370076 96.16563839655561) (end 103.67275319370076 96.16775319370076) (width 0.15) (layer F.Cu) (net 2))
 (segment (start 103.67275319370076 96.16775319370076) (end 103.8 96.295) (width 0.15) (layer F.Cu) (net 2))
 (segment (start 103.8 96.295) (end 106.44919149441102 96.295) (width 0.15) (layer B.Cu) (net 2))
 (segment (start 106.44919149441102 96.295) (end 108.1105838445991 97.95639235018807) (width 0.15) (layer B.Cu) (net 2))
 (segment (start 108.1105838445991 97.95639235018807) (end 108.25660764981193 97.95639235018807) (width 0.15) (layer B.Cu) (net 2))
 (segment (start 108.25660764981193 97.95639235018807) (end 108.27 97.943) (width 0.15) (layer B.Cu) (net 2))
 (segment (start 108.27 97.943) (end 109.667 99.34) (width 0.15) (layer F.Cu) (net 2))
 (segment (start 109.667 99.34) (end 110.96437019999988 99.33959999999996) (width 0.15) (layer F.Cu) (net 2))
 (gr_line (start 60 130) (end 140 130) (width 0.1) (layer Edge.Cuts))
 (gr_line (start 140 130) (end 140 70) (width 0.1) (layer Edge.Cuts))
 (gr_line (start 140 70) (end 60 70) (width 0.1) (layer Edge.Cuts))
 (gr_line (start 60 70) (end 60 130) (width 0.1) (layer Edge.Cuts))
 (via (at 102.085 82.132) (size 0.3) (drill 0.2) (layers F.Cu B.Cu) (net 7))
 (via (at 101.584 89.342) (size 0.3) (drill 0.2) (layers F.Cu B.Cu) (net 7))
 (via (at 100.952 83.959) (size 0.3) (drill 0.2) (layers F.Cu B.Cu) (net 6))
 (via (at 100.183 89.341) (size 0.3) (drill 0.2) (layers F.Cu B.Cu) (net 6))
 (via (at 98.016 91.538) (size 0.3) (drill 0.2) (layers F.Cu B.Cu) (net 1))
 (via (at 98.933 91.095) (size 0.3) (drill 0.2) (layers F.Cu B.Cu) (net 1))
 (via (at 104.126 92.17) (size 0.3) (drill 0.2) (layers F.Cu B.Cu) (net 1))
 (via (at 104.384 88.782) (size 0.3) (drill 0.2) (layers F.Cu B.Cu) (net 1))
 (via (at 103.8 96.295) (size 0.3) (drill 0.2) (layers F.Cu B.Cu) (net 2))
 (via (at 108.27 97.943) (size 0.3) (drill 0.2) (layers F.Cu B.Cu) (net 2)))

